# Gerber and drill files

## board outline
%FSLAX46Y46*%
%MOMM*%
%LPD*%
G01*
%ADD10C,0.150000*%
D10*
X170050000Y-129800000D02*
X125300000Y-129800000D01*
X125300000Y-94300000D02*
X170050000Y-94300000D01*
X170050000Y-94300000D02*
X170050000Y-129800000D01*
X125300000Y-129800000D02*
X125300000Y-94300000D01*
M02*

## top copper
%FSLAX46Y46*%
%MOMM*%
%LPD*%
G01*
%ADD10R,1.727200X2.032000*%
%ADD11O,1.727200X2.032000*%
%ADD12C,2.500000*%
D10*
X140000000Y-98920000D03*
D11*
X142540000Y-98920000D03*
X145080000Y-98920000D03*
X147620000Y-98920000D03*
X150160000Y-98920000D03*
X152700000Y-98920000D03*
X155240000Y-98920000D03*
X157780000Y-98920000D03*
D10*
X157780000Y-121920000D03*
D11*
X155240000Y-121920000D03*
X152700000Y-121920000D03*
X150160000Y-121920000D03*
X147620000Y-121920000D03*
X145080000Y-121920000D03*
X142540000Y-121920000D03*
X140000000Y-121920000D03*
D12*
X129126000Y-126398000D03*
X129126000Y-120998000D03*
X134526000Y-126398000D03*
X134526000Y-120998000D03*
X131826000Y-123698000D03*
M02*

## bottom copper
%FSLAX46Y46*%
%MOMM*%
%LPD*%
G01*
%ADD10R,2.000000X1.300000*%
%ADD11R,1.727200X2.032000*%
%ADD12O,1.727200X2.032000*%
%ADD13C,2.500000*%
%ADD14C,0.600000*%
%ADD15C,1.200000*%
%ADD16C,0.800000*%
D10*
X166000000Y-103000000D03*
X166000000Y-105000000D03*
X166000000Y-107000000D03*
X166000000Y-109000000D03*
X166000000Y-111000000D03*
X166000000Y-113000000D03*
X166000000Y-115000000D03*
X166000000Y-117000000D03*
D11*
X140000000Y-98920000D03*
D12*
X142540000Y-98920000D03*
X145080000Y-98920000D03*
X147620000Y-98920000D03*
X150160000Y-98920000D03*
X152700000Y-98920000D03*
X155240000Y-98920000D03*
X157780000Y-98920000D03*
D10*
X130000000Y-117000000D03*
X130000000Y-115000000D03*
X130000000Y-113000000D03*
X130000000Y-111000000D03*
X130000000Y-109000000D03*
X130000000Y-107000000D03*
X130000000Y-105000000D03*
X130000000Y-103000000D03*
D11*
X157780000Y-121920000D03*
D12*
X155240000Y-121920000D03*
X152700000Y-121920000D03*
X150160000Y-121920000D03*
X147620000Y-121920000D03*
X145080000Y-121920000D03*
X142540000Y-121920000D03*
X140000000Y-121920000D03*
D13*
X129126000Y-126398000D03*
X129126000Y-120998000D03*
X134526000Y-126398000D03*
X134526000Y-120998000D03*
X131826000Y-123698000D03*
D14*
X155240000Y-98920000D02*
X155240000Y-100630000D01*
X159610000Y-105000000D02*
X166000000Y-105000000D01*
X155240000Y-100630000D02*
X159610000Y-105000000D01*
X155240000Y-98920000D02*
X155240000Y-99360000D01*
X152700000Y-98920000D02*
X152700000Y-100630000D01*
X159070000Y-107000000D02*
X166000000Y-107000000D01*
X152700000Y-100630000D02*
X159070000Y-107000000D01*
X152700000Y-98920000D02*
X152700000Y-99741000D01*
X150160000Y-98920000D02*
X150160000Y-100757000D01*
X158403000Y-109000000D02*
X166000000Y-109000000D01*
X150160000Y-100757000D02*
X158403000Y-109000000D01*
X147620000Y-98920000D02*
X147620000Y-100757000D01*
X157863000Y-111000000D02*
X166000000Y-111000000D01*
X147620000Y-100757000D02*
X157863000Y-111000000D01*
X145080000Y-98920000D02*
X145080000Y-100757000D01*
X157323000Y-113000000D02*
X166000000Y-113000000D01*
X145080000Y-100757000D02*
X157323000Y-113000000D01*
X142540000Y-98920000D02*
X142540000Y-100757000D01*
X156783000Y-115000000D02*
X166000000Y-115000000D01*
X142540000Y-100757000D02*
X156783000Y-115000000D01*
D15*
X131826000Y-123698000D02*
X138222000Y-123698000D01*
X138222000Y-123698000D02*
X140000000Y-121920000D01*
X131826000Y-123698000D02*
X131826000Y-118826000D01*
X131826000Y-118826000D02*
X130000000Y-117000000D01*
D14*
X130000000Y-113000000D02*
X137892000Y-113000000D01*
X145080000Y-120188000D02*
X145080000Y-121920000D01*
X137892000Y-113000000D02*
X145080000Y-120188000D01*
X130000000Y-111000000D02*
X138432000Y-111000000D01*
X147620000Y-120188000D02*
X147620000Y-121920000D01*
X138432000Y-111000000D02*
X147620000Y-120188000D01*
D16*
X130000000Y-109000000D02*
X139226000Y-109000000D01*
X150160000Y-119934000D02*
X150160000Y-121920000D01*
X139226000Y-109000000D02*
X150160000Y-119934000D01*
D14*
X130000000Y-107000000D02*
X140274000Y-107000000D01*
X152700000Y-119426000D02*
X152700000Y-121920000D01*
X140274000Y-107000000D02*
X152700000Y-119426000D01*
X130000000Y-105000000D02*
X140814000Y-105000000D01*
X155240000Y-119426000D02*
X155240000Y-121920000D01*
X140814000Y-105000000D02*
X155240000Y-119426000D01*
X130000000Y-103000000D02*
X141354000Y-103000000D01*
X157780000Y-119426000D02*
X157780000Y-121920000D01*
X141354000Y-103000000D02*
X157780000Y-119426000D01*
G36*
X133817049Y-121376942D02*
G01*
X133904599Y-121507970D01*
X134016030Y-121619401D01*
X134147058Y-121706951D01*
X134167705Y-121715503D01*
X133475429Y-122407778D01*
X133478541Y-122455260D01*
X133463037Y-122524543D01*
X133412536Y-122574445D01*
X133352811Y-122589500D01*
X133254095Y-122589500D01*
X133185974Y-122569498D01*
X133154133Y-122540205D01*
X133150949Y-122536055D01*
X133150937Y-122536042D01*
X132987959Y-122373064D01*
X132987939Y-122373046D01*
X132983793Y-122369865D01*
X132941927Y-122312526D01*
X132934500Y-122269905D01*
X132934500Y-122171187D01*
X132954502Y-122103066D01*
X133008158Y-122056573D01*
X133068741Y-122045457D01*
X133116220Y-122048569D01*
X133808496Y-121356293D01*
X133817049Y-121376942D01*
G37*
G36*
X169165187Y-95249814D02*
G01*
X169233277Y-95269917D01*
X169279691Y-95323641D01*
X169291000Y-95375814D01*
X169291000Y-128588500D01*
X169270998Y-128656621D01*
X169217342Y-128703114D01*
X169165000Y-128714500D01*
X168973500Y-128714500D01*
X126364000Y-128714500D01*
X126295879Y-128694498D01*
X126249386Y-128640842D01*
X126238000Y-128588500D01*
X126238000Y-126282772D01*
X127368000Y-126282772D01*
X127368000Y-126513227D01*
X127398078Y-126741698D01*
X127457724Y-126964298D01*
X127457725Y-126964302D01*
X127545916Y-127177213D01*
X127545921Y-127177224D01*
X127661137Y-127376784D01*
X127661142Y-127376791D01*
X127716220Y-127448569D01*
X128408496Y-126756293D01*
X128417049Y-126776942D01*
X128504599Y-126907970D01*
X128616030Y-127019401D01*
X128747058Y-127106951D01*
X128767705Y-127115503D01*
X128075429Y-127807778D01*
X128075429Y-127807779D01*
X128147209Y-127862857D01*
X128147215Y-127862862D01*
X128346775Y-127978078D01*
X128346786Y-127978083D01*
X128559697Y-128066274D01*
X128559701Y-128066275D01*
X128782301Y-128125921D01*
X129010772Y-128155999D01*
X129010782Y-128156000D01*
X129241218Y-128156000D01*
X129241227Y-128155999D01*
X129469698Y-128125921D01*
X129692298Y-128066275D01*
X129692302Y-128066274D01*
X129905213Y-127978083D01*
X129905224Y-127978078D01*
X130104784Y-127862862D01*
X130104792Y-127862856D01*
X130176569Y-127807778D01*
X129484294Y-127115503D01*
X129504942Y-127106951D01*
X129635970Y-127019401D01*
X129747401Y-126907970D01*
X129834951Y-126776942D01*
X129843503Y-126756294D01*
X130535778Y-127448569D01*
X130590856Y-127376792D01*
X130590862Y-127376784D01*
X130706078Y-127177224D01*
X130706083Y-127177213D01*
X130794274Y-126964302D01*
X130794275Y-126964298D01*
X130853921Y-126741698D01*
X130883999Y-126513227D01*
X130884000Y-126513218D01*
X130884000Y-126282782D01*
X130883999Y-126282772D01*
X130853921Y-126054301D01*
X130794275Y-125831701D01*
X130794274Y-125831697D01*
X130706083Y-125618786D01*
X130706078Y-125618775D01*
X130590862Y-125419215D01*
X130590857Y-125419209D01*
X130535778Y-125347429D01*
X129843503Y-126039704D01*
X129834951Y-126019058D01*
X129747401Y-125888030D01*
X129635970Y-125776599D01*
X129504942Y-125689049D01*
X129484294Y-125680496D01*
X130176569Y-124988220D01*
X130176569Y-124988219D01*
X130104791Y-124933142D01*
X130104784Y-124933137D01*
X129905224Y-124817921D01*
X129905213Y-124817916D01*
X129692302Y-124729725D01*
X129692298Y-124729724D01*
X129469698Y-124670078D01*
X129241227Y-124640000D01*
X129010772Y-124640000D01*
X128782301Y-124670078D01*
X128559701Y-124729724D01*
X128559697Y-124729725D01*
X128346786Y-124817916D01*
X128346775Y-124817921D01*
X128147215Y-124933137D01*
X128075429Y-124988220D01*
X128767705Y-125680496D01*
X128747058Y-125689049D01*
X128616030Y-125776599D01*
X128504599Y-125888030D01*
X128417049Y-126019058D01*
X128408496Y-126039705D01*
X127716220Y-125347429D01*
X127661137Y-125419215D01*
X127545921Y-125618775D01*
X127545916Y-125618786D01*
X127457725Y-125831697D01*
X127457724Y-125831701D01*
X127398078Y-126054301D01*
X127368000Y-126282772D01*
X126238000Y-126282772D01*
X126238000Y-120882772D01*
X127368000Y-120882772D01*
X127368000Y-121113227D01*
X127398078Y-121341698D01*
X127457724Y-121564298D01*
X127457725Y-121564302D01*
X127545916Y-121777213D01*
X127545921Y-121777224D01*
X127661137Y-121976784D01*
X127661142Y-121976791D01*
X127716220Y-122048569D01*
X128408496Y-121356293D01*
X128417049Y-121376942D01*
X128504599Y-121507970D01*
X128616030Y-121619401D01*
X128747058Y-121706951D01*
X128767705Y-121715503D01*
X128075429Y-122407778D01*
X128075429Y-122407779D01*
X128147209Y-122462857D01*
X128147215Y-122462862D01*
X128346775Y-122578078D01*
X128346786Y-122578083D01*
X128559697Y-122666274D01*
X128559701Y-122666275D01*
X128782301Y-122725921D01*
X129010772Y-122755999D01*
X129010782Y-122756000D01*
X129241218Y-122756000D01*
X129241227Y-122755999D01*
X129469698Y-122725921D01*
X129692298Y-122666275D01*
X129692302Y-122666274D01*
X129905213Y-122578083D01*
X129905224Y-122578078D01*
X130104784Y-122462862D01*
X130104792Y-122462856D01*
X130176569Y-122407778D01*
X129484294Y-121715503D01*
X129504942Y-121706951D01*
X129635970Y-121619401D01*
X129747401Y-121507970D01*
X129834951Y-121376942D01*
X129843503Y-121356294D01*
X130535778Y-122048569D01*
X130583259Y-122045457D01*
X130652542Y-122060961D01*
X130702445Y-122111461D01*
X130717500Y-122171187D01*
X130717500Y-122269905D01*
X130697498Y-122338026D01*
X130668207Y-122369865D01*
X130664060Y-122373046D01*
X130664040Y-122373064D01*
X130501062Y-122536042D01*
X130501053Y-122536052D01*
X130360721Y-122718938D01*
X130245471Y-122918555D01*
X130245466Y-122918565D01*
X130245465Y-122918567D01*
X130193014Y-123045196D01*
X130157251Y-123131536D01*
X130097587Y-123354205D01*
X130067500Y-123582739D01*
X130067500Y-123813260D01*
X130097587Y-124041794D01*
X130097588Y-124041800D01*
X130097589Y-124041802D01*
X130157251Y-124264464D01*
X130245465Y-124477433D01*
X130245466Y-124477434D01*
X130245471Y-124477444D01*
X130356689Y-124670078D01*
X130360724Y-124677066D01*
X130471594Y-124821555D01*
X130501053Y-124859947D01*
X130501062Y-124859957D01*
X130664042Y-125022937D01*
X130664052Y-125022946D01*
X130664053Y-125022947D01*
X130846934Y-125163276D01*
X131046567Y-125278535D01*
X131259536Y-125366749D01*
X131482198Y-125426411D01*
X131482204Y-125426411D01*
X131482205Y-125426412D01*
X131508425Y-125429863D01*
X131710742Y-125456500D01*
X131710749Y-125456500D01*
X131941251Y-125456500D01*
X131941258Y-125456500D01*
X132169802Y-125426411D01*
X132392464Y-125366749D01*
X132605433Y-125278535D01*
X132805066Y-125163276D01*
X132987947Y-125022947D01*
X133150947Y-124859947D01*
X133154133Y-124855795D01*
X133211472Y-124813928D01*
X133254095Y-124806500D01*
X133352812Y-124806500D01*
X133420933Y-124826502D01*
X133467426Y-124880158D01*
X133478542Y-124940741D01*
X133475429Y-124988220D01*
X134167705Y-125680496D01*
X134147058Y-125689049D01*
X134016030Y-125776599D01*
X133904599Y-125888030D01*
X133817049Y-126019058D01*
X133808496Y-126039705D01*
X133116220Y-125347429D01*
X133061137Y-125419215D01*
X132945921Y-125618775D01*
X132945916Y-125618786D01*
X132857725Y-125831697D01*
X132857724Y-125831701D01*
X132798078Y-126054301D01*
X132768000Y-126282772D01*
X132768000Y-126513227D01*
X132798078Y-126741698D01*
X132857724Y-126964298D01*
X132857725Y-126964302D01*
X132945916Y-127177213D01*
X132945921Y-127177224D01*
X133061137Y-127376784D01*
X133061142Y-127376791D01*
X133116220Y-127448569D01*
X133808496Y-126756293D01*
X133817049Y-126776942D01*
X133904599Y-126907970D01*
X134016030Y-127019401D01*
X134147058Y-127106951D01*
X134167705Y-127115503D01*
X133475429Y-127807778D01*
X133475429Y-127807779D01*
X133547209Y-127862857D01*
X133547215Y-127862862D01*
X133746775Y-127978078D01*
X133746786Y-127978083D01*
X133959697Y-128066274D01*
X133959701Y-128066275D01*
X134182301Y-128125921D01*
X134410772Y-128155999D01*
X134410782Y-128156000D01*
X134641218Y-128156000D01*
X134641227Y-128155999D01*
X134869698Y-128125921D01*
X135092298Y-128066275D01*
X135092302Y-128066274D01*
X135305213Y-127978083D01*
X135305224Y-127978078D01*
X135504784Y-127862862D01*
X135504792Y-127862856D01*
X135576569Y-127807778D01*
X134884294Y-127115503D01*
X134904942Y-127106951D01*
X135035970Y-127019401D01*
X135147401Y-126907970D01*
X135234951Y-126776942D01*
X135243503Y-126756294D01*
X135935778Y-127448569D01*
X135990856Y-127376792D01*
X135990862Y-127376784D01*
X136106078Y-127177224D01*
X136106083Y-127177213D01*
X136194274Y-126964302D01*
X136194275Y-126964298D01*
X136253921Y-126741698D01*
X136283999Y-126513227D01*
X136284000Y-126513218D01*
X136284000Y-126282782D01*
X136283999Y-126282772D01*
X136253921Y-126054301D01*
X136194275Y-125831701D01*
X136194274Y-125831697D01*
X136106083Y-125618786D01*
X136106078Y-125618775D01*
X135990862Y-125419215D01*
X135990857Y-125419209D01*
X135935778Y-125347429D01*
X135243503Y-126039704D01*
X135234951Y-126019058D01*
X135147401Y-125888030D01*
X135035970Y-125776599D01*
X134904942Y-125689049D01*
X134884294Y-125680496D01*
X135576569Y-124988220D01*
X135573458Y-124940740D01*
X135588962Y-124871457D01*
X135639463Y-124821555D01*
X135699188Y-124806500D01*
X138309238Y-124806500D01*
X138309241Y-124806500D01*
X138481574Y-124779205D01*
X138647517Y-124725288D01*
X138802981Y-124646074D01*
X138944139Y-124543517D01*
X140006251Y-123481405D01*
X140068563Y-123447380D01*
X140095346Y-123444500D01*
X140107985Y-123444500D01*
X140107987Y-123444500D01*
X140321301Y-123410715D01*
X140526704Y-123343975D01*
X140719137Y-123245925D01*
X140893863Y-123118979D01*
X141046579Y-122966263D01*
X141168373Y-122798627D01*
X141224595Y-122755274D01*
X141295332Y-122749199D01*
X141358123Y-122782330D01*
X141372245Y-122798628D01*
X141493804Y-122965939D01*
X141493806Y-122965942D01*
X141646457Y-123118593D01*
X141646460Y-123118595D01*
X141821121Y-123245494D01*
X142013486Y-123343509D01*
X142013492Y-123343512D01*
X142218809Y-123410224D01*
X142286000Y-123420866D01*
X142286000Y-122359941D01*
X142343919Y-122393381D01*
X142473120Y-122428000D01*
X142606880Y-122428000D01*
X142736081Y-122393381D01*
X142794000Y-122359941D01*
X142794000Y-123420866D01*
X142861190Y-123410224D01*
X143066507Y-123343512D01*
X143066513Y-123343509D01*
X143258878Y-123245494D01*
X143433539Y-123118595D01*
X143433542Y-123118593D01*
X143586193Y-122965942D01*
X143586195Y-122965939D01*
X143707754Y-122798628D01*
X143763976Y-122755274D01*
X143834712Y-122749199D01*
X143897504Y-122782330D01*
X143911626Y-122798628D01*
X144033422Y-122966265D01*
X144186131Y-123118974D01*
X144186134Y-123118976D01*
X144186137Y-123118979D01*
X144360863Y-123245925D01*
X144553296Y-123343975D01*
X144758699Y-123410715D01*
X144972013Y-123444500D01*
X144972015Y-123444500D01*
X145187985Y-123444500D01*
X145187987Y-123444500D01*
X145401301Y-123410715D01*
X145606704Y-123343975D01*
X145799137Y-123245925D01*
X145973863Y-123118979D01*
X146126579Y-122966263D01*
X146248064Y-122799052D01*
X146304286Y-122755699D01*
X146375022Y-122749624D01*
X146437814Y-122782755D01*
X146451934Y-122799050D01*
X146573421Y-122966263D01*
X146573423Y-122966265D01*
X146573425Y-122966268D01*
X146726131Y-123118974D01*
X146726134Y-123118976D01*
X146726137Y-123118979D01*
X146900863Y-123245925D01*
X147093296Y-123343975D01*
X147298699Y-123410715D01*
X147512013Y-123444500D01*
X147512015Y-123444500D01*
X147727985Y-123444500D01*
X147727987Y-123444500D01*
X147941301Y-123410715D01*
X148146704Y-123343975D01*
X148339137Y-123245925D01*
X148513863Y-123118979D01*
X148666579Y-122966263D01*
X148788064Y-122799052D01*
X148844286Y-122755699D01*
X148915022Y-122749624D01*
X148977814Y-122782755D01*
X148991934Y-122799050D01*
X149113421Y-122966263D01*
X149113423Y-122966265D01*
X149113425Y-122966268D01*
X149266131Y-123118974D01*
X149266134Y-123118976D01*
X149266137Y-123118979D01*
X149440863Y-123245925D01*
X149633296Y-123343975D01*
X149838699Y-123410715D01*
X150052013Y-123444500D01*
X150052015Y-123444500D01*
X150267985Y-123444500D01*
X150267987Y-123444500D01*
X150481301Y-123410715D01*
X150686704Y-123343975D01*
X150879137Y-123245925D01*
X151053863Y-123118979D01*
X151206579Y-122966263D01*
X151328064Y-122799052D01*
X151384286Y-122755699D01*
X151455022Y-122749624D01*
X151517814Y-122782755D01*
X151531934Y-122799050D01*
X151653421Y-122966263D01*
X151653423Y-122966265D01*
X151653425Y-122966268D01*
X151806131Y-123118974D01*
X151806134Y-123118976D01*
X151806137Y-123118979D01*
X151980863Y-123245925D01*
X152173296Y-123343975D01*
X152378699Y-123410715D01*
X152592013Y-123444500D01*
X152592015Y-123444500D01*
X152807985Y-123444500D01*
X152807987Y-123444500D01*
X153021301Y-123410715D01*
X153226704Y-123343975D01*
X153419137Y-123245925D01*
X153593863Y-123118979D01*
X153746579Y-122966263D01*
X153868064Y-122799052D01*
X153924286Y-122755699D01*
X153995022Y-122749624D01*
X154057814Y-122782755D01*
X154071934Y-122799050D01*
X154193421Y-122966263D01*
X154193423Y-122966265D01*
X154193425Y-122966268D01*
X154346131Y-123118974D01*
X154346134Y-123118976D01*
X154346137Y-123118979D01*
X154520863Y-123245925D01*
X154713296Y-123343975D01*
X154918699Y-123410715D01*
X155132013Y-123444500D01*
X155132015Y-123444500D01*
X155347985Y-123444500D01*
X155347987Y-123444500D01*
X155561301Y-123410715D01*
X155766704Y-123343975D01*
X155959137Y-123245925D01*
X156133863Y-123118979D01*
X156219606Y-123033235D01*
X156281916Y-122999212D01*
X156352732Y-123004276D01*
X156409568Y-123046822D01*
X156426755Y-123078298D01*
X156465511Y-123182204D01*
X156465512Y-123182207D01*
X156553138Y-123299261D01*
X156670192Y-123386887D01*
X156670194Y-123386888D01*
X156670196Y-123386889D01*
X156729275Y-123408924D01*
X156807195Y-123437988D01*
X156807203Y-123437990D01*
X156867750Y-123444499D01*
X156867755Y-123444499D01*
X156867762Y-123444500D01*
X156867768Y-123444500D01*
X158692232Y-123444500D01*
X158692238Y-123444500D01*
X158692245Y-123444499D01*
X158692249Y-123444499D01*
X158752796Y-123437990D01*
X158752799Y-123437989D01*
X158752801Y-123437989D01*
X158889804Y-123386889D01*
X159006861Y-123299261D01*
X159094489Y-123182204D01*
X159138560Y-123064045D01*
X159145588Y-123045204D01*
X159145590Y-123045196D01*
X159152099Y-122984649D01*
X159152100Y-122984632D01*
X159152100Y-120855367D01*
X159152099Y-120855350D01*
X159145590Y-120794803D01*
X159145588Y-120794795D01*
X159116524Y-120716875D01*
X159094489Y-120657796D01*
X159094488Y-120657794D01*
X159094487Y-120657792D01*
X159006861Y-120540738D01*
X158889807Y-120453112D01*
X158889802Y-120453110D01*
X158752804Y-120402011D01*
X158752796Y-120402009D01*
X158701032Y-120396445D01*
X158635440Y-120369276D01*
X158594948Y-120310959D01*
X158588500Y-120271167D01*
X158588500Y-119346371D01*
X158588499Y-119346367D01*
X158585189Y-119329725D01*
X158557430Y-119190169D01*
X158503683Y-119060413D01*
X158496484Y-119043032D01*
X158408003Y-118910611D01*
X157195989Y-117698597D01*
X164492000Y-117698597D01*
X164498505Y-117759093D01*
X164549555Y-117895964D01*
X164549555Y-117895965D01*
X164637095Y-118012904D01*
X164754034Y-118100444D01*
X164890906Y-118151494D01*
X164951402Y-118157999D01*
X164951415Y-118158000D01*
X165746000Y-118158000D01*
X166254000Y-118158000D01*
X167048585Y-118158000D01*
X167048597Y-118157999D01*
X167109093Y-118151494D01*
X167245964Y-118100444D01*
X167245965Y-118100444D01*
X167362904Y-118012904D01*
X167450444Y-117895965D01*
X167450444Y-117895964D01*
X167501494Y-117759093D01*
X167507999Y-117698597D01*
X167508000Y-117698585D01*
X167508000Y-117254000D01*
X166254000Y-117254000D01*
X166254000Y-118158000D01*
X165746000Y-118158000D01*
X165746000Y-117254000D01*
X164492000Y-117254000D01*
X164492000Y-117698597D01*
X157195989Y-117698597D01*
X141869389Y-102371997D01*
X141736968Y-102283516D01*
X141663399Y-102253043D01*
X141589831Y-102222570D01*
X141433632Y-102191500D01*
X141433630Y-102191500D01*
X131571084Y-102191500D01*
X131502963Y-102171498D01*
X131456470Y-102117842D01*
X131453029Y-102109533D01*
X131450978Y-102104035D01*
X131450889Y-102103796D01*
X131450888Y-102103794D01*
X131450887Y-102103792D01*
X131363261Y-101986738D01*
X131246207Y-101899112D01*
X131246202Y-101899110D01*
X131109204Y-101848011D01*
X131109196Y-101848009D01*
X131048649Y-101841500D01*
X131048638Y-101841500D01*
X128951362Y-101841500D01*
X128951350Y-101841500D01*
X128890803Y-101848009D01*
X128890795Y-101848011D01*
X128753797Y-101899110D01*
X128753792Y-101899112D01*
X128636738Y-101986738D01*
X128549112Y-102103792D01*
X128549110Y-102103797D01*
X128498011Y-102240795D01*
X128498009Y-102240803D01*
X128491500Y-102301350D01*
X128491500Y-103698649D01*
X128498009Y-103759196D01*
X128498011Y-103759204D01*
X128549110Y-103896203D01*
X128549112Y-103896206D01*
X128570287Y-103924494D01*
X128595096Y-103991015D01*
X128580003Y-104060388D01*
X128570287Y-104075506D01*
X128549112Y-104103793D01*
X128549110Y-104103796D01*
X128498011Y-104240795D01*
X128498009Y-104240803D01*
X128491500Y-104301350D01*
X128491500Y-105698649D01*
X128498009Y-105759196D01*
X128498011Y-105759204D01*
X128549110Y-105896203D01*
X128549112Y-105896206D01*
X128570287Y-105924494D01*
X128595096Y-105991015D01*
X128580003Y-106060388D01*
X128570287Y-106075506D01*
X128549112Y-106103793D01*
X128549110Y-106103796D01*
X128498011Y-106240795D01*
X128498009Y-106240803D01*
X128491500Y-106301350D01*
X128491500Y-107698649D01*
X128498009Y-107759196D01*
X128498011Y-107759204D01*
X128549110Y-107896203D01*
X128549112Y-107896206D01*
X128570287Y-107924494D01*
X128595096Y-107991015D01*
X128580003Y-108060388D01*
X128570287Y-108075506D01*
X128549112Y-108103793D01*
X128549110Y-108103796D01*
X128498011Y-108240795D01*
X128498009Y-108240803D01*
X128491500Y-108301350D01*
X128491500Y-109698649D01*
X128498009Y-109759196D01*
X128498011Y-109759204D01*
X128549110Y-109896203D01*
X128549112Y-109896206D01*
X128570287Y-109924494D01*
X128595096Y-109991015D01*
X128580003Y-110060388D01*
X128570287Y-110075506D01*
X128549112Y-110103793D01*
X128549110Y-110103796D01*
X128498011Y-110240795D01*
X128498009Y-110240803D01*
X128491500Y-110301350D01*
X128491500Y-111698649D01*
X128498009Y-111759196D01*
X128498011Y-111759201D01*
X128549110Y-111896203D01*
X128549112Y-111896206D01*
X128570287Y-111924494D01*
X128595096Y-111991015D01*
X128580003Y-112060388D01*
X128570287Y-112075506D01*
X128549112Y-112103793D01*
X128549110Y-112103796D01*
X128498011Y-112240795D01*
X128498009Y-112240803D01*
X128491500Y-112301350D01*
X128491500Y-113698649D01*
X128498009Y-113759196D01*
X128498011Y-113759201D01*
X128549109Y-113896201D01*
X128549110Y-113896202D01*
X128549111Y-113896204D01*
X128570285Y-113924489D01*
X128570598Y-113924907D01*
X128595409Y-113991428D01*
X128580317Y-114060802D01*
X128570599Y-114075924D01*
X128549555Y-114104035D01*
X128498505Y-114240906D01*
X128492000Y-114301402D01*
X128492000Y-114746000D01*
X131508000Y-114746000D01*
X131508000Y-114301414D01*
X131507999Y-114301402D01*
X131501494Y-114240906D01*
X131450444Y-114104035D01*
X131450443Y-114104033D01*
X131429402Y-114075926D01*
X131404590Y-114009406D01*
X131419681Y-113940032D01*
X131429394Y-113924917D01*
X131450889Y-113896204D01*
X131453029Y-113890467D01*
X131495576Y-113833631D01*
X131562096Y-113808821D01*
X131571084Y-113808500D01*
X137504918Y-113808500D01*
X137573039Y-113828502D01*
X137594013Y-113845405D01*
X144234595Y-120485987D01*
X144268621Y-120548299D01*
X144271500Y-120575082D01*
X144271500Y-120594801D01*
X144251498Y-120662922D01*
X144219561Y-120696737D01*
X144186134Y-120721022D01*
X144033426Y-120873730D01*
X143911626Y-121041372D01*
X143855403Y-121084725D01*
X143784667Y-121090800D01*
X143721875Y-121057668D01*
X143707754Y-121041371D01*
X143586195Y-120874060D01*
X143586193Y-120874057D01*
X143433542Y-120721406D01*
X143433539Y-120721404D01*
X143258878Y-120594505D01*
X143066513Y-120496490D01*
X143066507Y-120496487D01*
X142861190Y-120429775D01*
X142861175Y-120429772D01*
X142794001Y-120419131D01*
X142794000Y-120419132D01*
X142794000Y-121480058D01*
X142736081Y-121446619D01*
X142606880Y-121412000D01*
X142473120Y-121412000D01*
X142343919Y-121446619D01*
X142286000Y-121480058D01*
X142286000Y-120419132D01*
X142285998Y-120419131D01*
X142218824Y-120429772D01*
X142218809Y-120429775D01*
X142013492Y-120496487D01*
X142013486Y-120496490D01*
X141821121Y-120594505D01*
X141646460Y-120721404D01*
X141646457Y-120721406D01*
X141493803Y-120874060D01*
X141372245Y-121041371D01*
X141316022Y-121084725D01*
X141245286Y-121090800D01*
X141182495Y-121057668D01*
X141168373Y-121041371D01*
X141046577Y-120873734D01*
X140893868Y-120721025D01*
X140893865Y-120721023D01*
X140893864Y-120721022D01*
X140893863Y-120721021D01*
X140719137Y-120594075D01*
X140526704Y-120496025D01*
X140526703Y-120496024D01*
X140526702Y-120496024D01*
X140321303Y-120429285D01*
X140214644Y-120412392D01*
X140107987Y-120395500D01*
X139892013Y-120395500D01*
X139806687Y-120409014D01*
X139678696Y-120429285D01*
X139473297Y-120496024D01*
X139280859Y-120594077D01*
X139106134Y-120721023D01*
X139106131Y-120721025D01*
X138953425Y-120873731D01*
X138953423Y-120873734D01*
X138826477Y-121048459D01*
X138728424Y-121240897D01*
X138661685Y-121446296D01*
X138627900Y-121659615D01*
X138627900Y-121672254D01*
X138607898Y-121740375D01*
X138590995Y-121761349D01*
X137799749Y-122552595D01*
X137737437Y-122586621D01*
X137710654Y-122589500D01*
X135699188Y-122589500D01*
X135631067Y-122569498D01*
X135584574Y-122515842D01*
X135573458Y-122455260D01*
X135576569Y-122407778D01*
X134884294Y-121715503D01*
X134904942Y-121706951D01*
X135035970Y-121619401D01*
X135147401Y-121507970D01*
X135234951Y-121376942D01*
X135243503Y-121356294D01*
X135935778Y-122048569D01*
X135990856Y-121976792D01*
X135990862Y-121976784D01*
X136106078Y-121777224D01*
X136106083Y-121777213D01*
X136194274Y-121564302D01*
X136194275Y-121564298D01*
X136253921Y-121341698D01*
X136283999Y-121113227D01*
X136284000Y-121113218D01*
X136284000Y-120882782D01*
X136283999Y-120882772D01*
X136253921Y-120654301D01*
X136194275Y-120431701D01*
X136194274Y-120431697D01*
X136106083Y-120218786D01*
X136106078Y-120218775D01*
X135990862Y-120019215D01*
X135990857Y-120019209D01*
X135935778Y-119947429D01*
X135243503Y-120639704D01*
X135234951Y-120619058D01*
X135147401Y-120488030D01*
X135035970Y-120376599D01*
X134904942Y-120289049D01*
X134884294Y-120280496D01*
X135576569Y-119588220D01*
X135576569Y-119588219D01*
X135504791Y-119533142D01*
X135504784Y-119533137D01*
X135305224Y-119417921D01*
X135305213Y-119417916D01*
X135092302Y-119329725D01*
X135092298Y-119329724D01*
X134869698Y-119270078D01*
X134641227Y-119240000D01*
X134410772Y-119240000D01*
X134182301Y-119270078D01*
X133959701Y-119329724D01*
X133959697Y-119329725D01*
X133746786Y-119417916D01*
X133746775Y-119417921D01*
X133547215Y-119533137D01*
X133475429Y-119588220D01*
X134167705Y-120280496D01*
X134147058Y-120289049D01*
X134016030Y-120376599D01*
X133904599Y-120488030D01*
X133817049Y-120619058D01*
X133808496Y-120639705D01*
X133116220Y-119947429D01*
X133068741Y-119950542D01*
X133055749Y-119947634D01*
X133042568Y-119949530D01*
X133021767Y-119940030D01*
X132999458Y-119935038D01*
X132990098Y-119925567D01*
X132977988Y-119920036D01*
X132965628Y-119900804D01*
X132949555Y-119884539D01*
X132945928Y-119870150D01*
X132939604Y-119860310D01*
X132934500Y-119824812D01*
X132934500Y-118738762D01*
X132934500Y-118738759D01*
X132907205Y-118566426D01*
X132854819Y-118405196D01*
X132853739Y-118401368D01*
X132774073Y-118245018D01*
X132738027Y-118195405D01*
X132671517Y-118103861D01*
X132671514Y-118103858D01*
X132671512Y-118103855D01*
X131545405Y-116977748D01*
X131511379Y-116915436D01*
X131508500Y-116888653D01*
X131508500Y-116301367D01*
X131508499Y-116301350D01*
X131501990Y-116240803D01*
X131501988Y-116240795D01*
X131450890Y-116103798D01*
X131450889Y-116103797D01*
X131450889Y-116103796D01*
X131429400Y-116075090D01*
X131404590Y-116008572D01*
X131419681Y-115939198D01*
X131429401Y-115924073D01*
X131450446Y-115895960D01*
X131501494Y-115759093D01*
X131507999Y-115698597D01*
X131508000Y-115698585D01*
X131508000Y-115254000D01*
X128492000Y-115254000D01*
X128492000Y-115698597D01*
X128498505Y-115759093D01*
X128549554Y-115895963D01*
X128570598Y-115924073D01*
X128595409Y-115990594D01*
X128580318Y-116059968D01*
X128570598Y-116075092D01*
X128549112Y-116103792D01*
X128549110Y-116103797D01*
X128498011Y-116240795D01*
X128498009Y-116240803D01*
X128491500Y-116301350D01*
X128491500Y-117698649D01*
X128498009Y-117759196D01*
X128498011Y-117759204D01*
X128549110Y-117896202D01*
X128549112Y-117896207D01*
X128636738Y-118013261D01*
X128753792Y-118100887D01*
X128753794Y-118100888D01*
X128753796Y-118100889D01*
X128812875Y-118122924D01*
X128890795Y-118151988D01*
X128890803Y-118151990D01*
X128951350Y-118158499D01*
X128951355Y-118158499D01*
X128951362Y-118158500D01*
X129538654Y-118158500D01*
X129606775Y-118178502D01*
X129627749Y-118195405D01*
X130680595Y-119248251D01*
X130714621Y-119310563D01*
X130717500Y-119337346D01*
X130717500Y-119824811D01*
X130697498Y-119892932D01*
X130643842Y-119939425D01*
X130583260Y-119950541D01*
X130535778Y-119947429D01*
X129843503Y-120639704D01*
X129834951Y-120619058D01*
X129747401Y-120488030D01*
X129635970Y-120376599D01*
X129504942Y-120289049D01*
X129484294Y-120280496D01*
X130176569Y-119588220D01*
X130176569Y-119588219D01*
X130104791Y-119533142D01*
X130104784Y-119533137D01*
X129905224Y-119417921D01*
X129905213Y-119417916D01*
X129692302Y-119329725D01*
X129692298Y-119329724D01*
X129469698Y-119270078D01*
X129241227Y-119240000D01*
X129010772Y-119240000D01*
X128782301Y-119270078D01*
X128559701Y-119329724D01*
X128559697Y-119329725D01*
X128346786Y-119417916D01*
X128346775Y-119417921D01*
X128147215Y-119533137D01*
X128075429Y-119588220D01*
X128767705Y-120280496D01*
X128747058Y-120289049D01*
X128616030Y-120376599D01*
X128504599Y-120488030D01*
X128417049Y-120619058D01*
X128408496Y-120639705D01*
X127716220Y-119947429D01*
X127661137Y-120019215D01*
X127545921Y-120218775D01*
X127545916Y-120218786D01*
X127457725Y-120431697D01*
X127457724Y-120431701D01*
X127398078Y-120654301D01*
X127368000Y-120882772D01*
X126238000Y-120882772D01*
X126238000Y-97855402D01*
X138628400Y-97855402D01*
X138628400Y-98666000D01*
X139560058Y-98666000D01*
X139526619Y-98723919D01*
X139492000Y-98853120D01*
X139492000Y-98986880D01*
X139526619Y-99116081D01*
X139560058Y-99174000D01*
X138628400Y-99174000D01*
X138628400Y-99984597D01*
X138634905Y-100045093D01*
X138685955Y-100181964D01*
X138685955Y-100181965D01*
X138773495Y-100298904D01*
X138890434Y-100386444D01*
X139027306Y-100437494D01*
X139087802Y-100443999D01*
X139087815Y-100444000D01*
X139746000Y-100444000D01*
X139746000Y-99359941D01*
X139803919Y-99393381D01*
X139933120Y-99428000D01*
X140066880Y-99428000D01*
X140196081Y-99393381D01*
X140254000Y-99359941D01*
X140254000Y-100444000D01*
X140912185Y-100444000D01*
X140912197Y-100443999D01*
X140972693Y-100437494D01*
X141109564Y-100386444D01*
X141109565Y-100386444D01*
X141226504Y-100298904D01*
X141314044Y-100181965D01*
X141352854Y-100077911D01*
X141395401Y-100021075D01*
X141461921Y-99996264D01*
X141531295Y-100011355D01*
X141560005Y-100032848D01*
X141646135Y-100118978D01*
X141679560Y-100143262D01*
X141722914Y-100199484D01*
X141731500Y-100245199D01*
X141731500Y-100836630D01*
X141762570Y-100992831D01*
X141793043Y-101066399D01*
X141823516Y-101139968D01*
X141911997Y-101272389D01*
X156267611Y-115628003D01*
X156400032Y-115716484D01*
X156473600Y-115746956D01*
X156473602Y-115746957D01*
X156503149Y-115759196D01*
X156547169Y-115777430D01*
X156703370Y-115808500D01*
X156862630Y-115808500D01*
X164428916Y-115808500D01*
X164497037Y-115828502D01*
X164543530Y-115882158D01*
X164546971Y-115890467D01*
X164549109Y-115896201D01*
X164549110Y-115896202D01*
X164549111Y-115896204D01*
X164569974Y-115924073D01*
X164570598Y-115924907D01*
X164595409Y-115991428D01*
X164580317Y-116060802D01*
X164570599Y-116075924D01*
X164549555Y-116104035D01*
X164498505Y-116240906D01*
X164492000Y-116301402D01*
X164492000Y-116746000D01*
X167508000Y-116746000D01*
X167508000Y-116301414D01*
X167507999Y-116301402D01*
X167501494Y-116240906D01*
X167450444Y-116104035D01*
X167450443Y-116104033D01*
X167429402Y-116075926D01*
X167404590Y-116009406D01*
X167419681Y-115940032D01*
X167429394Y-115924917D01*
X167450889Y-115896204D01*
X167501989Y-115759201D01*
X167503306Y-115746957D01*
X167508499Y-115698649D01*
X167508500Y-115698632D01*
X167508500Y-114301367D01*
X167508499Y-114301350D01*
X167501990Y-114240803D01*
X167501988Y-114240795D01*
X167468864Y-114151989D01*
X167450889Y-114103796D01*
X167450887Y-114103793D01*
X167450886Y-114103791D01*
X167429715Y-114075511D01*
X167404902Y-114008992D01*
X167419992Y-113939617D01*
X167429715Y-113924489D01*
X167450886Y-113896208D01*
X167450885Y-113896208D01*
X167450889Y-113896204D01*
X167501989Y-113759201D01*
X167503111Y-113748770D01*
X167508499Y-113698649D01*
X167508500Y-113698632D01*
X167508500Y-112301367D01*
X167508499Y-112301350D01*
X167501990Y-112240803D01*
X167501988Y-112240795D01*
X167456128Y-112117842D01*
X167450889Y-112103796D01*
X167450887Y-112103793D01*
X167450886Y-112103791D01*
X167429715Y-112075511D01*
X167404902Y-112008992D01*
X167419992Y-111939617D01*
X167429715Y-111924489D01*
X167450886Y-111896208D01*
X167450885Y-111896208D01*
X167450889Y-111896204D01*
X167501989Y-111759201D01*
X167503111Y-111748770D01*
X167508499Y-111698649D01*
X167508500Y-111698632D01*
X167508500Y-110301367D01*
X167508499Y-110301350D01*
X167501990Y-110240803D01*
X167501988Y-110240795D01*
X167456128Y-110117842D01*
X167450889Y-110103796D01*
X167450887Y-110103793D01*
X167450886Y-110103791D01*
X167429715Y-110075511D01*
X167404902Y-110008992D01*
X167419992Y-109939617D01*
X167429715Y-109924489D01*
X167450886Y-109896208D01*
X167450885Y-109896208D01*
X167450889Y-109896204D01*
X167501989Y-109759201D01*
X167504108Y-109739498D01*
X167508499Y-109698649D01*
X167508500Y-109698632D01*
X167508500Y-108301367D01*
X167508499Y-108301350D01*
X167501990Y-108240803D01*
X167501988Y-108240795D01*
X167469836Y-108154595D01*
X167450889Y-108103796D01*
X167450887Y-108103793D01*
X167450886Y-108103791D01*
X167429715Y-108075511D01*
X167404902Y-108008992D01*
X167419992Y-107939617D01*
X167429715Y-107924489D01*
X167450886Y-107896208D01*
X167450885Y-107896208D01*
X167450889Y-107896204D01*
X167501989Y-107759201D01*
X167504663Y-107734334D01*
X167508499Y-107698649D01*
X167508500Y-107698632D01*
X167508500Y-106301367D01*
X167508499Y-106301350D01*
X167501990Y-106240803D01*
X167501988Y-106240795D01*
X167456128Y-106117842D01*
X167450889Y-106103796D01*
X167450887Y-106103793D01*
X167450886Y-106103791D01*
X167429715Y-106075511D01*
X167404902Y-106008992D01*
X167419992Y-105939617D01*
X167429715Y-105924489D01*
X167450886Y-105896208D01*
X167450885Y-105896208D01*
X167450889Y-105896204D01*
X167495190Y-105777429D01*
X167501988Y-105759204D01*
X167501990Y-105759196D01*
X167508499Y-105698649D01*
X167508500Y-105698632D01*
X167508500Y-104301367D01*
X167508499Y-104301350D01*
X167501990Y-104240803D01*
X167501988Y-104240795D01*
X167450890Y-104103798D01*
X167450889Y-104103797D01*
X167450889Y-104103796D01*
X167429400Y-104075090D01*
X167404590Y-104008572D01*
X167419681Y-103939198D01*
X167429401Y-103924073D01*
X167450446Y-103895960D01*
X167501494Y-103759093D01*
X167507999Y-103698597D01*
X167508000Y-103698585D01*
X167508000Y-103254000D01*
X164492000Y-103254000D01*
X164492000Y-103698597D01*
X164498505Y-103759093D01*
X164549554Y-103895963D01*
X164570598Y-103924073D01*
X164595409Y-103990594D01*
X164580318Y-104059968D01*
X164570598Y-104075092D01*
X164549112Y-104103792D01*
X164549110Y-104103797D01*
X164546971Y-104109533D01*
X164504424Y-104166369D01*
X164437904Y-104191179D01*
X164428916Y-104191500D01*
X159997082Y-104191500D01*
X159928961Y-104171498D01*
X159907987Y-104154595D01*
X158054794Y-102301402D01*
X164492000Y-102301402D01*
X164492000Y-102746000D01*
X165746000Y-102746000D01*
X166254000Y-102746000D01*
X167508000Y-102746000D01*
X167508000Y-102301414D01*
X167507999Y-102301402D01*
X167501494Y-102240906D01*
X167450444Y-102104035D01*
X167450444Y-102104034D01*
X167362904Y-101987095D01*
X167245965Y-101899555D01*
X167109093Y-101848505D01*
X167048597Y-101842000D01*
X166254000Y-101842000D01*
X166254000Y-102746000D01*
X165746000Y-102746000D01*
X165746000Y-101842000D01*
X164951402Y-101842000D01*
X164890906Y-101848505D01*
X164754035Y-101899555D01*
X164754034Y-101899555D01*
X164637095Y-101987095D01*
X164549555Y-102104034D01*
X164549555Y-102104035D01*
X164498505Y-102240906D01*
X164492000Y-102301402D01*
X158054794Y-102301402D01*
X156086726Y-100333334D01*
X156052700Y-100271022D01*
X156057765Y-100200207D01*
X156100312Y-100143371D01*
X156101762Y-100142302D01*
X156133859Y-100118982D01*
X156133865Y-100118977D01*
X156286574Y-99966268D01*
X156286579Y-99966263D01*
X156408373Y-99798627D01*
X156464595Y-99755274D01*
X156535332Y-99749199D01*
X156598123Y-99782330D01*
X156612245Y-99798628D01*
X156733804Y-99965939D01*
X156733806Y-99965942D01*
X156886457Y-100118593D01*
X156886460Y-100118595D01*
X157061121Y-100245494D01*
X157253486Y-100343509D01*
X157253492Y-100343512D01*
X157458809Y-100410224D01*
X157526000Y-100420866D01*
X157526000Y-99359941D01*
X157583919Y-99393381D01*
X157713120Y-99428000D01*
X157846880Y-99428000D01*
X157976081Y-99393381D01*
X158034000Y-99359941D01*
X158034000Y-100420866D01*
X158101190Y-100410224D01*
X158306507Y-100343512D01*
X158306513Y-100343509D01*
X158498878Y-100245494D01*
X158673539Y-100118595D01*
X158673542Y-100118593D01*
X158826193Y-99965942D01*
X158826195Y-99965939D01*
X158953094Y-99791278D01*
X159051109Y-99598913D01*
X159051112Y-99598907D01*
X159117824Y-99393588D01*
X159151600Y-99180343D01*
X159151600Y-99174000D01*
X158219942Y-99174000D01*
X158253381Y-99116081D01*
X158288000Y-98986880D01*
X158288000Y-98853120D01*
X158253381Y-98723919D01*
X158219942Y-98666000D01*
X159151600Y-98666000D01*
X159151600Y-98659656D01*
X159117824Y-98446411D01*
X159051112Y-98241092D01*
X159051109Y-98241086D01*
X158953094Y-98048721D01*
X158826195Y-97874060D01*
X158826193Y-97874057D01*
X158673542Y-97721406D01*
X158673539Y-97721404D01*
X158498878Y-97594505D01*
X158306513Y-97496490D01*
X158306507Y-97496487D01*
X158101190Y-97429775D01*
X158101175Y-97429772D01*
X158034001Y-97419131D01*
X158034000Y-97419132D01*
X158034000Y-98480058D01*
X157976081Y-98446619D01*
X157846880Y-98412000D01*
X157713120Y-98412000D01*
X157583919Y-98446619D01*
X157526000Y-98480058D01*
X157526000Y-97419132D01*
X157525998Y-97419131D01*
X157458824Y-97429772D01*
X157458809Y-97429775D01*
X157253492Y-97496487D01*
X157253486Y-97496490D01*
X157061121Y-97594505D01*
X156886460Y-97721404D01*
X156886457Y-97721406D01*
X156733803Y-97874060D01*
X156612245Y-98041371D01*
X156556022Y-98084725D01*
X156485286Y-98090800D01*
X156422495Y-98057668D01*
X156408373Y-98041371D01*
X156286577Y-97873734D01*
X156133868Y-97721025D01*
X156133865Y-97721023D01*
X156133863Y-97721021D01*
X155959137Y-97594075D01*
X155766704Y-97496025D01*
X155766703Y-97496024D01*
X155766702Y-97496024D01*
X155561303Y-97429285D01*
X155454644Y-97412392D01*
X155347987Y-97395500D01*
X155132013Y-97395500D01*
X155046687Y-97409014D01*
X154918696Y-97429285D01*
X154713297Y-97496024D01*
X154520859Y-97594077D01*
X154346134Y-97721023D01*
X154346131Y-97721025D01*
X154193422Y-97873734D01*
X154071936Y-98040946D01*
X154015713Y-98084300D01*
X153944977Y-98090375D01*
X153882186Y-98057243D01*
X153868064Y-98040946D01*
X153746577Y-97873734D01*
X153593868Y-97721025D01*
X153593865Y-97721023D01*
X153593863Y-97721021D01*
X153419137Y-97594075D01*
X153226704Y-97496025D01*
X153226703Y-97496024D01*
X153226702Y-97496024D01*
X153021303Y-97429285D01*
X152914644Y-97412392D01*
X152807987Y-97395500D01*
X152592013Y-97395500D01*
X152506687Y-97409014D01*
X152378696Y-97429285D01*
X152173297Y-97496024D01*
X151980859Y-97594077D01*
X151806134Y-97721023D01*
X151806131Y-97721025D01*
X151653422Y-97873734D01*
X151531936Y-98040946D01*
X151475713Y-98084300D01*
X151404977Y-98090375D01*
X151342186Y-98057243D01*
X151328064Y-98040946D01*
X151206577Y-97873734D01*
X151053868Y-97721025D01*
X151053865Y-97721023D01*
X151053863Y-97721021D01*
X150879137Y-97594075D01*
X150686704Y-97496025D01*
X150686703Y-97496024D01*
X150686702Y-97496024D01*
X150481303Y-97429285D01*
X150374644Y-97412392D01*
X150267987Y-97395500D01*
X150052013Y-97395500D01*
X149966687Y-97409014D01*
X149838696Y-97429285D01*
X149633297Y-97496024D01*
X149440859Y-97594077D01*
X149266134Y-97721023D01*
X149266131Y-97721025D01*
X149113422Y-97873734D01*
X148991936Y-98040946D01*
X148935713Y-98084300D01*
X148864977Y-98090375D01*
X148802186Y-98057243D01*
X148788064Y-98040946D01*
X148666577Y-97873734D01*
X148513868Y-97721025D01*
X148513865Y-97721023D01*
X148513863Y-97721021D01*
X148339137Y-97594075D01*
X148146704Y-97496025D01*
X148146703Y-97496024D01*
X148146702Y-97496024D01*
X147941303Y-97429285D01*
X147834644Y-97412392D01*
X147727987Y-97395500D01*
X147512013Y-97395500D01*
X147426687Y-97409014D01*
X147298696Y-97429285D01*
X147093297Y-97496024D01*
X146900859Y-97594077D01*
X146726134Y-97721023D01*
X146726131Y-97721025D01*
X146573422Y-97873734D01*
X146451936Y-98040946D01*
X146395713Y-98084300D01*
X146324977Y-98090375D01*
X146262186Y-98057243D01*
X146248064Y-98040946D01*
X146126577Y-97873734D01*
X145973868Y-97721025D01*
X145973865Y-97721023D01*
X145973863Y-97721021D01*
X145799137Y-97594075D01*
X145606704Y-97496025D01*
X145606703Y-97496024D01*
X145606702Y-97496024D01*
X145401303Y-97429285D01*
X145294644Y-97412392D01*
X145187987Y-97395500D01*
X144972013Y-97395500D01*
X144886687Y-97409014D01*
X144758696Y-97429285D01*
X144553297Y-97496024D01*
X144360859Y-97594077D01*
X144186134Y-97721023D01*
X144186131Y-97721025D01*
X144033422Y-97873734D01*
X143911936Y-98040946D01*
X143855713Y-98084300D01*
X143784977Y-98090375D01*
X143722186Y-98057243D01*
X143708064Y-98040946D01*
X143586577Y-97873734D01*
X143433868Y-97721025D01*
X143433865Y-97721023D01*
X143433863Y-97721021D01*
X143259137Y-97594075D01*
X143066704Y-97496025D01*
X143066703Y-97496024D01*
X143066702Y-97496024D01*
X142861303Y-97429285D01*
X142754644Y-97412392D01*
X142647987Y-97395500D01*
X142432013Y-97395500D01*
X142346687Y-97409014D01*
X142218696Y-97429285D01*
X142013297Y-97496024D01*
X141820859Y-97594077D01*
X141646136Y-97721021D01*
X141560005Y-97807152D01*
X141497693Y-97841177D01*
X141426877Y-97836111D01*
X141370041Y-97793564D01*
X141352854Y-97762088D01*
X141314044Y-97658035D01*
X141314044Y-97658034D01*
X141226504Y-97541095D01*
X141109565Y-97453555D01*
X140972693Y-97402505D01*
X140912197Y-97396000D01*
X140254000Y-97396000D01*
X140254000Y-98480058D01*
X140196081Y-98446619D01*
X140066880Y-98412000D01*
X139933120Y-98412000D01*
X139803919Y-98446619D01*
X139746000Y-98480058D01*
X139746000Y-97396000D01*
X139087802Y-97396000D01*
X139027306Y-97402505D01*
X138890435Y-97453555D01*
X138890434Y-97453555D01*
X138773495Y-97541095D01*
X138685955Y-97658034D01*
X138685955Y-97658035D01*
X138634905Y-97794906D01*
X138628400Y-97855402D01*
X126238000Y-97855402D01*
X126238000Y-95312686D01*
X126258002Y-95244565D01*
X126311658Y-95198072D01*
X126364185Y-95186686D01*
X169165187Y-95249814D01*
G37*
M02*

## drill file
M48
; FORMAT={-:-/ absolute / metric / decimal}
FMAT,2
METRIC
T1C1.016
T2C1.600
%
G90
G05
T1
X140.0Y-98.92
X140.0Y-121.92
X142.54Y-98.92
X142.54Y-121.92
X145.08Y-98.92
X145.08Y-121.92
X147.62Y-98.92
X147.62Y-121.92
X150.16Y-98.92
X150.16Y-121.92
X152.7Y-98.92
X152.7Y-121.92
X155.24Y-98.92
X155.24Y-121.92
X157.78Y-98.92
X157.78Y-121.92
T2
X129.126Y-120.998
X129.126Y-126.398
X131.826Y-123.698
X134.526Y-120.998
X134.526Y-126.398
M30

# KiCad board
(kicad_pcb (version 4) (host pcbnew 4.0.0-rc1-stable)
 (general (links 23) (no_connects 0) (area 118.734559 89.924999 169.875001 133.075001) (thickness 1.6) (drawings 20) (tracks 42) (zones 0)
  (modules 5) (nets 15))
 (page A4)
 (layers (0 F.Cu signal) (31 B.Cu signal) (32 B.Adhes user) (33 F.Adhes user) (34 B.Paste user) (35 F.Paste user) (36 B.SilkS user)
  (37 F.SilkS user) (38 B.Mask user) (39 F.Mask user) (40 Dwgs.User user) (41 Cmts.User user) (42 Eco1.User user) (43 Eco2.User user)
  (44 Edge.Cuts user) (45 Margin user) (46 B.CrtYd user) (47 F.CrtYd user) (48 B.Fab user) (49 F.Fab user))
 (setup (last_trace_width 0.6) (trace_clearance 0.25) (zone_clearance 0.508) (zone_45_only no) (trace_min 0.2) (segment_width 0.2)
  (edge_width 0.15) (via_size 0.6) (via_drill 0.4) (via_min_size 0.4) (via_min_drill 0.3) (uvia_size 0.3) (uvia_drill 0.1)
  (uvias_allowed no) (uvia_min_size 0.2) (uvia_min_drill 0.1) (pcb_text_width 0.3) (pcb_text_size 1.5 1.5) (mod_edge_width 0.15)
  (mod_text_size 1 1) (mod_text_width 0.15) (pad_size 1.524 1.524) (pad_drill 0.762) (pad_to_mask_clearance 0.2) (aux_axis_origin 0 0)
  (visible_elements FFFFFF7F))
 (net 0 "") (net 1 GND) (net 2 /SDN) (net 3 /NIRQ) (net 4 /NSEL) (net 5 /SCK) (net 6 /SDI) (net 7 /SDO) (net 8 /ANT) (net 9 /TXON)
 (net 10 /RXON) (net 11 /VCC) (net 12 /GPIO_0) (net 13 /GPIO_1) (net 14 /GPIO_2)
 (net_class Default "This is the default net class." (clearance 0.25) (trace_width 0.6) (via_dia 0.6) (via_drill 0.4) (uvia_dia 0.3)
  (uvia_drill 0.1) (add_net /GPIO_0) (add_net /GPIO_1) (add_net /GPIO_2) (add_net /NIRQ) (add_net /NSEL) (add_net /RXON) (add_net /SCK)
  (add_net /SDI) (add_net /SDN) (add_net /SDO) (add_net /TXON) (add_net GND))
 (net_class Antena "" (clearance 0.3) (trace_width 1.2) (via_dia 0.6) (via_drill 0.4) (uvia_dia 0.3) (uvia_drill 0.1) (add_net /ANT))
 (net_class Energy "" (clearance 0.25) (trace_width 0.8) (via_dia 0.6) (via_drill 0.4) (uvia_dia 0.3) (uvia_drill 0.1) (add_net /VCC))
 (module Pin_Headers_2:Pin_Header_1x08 (layer B.Cu) (at 166 110 90)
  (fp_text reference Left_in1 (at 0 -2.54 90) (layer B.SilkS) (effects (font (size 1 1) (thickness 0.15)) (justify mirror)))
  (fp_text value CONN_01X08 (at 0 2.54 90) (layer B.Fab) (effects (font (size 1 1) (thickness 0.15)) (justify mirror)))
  (pad 8 smd rect (at 7 0 90) (size 1.3 2) (layers B.Cu B.Paste B.Mask) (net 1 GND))
  (pad 7 smd rect (at 5 0 90) (size 1.3 2) (layers B.Cu B.Paste B.Mask) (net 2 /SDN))
  (pad 6 smd rect (at 3 0 90) (size 1.3 2) (layers B.Cu B.Paste B.Mask) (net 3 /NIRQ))
  (pad 5 smd rect (at 1 0 90) (size 1.3 2) (layers B.Cu B.Paste B.Mask) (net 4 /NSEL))
  (pad 4 smd rect (at -1 0 90) (size 1.3 2) (layers B.Cu B.Paste B.Mask) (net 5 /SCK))
  (pad 3 smd rect (at -3 0 90) (size 1.3 2) (layers B.Cu B.Paste B.Mask) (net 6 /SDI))
  (pad 2 smd rect (at -5 0 90) (size 1.3 2) (layers B.Cu B.Paste B.Mask) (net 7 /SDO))
  (pad 1 smd rect (at -7 0 90) (size 1.3 2) (layers B.Cu B.Paste B.Mask) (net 1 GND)))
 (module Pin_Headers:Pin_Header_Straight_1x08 (layer F.Cu) (at 140 98.92 90)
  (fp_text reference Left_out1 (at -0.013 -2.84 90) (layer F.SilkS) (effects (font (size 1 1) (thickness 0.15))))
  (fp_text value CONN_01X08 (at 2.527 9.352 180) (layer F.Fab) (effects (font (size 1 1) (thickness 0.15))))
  (pad 1 thru_hole rect (at 0 0 90) (size 2.032 1.7272) (drill 1.016) (layers *.Cu *.Mask F.SilkS) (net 1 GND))
  (pad 2 thru_hole oval (at 0 2.54 90) (size 2.032 1.7272) (drill 1.016) (layers *.Cu *.Mask F.SilkS) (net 7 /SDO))
  (pad 3 thru_hole oval (at 0 5.08 90) (size 2.032 1.7272) (drill 1.016) (layers *.Cu *.Mask F.SilkS) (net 6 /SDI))
  (pad 4 thru_hole oval (at 0 7.62 90) (size 2.032 1.7272) (drill 1.016) (layers *.Cu *.Mask F.SilkS) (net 5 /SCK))
  (pad 5 thru_hole oval (at 0 10.16 90) (size 2.032 1.7272) (drill 1.016) (layers *.Cu *.Mask F.SilkS) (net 4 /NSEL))
  (pad 6 thru_hole oval (at 0 12.7 90) (size 2.032 1.7272) (drill 1.016) (layers *.Cu *.Mask F.SilkS) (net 3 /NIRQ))
  (pad 7 thru_hole oval (at 0 15.24 90) (size 2.032 1.7272) (drill 1.016) (layers *.Cu *.Mask F.SilkS) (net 2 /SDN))
  (pad 8 thru_hole oval (at 0 17.78 90) (size 2.032 1.7272) (drill 1.016) (layers *.Cu *.Mask F.SilkS) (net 1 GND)))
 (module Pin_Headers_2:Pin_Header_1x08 (layer B.Cu) (at 130 110 270)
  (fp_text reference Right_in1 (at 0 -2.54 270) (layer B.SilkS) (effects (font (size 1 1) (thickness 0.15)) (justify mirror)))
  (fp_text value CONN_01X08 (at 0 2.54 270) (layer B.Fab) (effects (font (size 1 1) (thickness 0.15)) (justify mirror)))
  (pad 8 smd rect (at 7 0 270) (size 1.3 2) (layers B.Cu B.Paste B.Mask) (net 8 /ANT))
  (pad 7 smd rect (at 5 0 270) (size 1.3 2) (layers B.Cu B.Paste B.Mask) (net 1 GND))
  (pad 6 smd rect (at 3 0 270) (size 1.3 2) (layers B.Cu B.Paste B.Mask) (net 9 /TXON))
  (pad 5 smd rect (at 1 0 270) (size 1.3 2) (layers B.Cu B.Paste B.Mask) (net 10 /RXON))
  (pad 4 smd rect (at -1 0 270) (size 1.3 2) (layers B.Cu B.Paste B.Mask) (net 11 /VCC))
  (pad 3 smd rect (at -3 0 270) (size 1.3 2) (layers B.Cu B.Paste B.Mask) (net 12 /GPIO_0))
  (pad 2 smd rect (at -5 0 270) (size 1.3 2) (layers B.Cu B.Paste B.Mask) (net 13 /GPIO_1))
  (pad 1 smd rect (at -7 0 270) (size 1.3 2) (layers B.Cu B.Paste B.Mask) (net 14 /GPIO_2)))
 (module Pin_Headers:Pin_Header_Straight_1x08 (layer F.Cu) (at 157.78 121.92 270)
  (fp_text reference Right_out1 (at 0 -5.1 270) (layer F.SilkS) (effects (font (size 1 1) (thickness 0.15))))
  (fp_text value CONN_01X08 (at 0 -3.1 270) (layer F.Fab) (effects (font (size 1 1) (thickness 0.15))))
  (pad 1 thru_hole rect (at 0 0 270) (size 2.032 1.7272) (drill 1.016) (layers *.Cu *.Mask F.SilkS) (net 14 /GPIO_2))
  (pad 2 thru_hole oval (at 0 2.54 270) (size 2.032 1.7272) (drill 1.016) (layers *.Cu *.Mask F.SilkS) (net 13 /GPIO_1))
  (pad 3 thru_hole oval (at 0 5.08 270) (size 2.032 1.7272) (drill 1.016) (layers *.Cu *.Mask F.SilkS) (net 12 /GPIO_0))
  (pad 4 thru_hole oval (at 0 7.62 270) (size 2.032 1.7272) (drill 1.016) (layers *.Cu *.Mask F.SilkS) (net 11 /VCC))
  (pad 5 thru_hole oval (at 0 10.16 270) (size 2.032 1.7272) (drill 1.016) (layers *.Cu *.Mask F.SilkS) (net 10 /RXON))
  (pad 6 thru_hole oval (at 0 12.7 270) (size 2.032 1.7272) (drill 1.016) (layers *.Cu *.Mask F.SilkS) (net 9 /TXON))
  (pad 7 thru_hole oval (at 0 15.24 270) (size 2.032 1.7272) (drill 1.016) (layers *.Cu *.Mask F.SilkS) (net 1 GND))
  (pad 8 thru_hole oval (at 0 17.78 270) (size 2.032 1.7272) (drill 1.016) (layers *.Cu *.Mask F.SilkS) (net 8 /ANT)))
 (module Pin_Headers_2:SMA (layer F.Cu) (at 131.826 123.698 90)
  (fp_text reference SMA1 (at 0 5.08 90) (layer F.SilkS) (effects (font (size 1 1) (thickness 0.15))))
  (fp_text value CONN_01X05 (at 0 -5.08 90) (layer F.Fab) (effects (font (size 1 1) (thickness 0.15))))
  (pad 2 thru_hole circle (at -2.7 -2.7 90) (size 2.5 2.5) (drill 1.6) (layers *.Cu *.Mask F.SilkS) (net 1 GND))
  (pad 3 thru_hole circle (at 2.7 -2.7 90) (size 2.5 2.5) (drill 1.6) (layers *.Cu *.Mask F.SilkS) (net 1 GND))
  (pad 5 thru_hole circle (at -2.7 2.7 90) (size 2.5 2.5) (drill 1.6) (layers *.Cu *.Mask F.SilkS) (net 1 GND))
  (pad 4 thru_hole circle (at 2.7 2.7 90) (size 2.5 2.5) (drill 1.6) (layers *.Cu *.Mask F.SilkS) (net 1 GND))
  (pad 1 thru_hole circle (at 0 0 90) (size 2.5 2.5) (drill 1.6) (layers *.Cu *.Mask F.SilkS) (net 8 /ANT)))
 (gr_line (start 170.05 129.8) (end 125.3 129.8) (angle 90) (layer Edge.Cuts) (width 0.15))
 (gr_line (start 125.3 94.3) (end 170.05 94.3) (angle 90) (layer Edge.Cuts) (width 0.15))
 (gr_line (start 170.05 94.3) (end 170.05 129.8) (angle 90) (layer Edge.Cuts) (width 0.15))
 (gr_line (start 125.3 129.8) (end 125.3 94.3) (angle 90) (layer Edge.Cuts) (width 0.15))
 (segment (start 155.24 98.92) (end 155.24 100.63) (width 0.6) (layer B.Cu) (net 2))
 (segment (start 159.61 105) (end 166 105) (width 0.6) (layer B.Cu) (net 2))
 (segment (start 155.24 100.63) (end 159.61 105) (width 0.6) (layer B.Cu) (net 2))
 (segment (start 155.24 98.92) (end 155.24 99.36) (width 0.6) (layer B.Cu) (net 2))
 (segment (start 152.7 98.92) (end 152.7 100.63) (width 0.6) (layer B.Cu) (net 3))
 (segment (start 159.07 107) (end 166 107) (width 0.6) (layer B.Cu) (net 3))
 (segment (start 152.7 100.63) (end 159.07 107) (width 0.6) (layer B.Cu) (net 3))
 (segment (start 152.7 98.92) (end 152.7 99.741) (width 0.6) (layer B.Cu) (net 3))
 (segment (start 150.16 98.92) (end 150.16 100.757) (width 0.6) (layer B.Cu) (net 4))
 (segment (start 158.403 109) (end 166 109) (width 0.6) (layer B.Cu) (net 4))
 (segment (start 150.16 100.757) (end 158.403 109) (width 0.6) (layer B.Cu) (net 4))
 (segment (start 147.62 98.92) (end 147.62 100.757) (width 0.6) (layer B.Cu) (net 5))
 (segment (start 157.863 111) (end 166 111) (width 0.6) (layer B.Cu) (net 5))
 (segment (start 147.62 100.757) (end 157.863 111) (width 0.6) (layer B.Cu) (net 5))
 (segment (start 145.08 98.92) (end 145.08 100.757) (width 0.6) (layer B.Cu) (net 6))
 (segment (start 157.323 113) (end 166 113) (width 0.6) (layer B.Cu) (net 6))
 (segment (start 145.08 100.757) (end 157.323 113) (width 0.6) (layer B.Cu) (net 6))
 (segment (start 142.54 98.92) (end 142.54 100.757) (width 0.6) (layer B.Cu) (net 7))
 (segment (start 156.783 115) (end 166 115) (width 0.6) (layer B.Cu) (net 7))
 (segment (start 142.54 100.757) (end 156.783 115) (width 0.6) (layer B.Cu) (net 7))
 (segment (start 131.826 123.698) (end 138.222 123.698) (width 1.2) (layer B.Cu) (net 8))
 (segment (start 138.222 123.698) (end 140 121.92) (width 1.2) (layer B.Cu) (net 8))
 (segment (start 131.826 123.698) (end 131.826 118.826) (width 1.2) (layer B.Cu) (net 8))
 (segment (start 131.826 118.826) (end 130 117) (width 1.2) (layer B.Cu) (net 8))
 (segment (start 130 113) (end 137.892 113) (width 0.6) (layer B.Cu) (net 9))
 (segment (start 145.08 120.188) (end 145.08 121.92) (width 0.6) (layer B.Cu) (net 9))
 (segment (start 137.892 113) (end 145.08 120.188) (width 0.6) (layer B.Cu) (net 9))
 (segment (start 130 111) (end 138.432 111) (width 0.6) (layer B.Cu) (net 10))
 (segment (start 147.62 120.188) (end 147.62 121.92) (width 0.6) (layer B.Cu) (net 10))
 (segment (start 138.432 111) (end 147.62 120.188) (width 0.6) (layer B.Cu) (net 10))
 (segment (start 130 109) (end 139.226 109) (width 0.8) (layer B.Cu) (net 11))
 (segment (start 150.16 119.934) (end 150.16 121.92) (width 0.8) (layer B.Cu) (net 11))
 (segment (start 139.226 109) (end 150.16 119.934) (width 0.8) (layer B.Cu) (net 11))
 (segment (start 130 107) (end 140.274 107) (width 0.6) (layer B.Cu) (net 12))
 (segment (start 152.7 119.426) (end 152.7 121.92) (width 0.6) (layer B.Cu) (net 12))
 (segment (start 140.274 107) (end 152.7 119.426) (width 0.6) (layer B.Cu) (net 12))
 (segment (start 130 105) (end 140.814 105) (width 0.6) (layer B.Cu) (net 13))
 (segment (start 155.24 119.426) (end 155.24 121.92) (width 0.6) (layer B.Cu) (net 13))
 (segment (start 140.814 105) (end 155.24 119.426) (width 0.6) (layer B.Cu) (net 13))
 (segment (start 130 103) (end 141.354 103) (width 0.6) (layer B.Cu) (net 14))
 (segment (start 157.78 119.426) (end 157.78 121.92) (width 0.6) (layer B.Cu) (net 14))
 (segment (start 141.354 103) (end 157.78 119.426) (width 0.6) (layer B.Cu) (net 14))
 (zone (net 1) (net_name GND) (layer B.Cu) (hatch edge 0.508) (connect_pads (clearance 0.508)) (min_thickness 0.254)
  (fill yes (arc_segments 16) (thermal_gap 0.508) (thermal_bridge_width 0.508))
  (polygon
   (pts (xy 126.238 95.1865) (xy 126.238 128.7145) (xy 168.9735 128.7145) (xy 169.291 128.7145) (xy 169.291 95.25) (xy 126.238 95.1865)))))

